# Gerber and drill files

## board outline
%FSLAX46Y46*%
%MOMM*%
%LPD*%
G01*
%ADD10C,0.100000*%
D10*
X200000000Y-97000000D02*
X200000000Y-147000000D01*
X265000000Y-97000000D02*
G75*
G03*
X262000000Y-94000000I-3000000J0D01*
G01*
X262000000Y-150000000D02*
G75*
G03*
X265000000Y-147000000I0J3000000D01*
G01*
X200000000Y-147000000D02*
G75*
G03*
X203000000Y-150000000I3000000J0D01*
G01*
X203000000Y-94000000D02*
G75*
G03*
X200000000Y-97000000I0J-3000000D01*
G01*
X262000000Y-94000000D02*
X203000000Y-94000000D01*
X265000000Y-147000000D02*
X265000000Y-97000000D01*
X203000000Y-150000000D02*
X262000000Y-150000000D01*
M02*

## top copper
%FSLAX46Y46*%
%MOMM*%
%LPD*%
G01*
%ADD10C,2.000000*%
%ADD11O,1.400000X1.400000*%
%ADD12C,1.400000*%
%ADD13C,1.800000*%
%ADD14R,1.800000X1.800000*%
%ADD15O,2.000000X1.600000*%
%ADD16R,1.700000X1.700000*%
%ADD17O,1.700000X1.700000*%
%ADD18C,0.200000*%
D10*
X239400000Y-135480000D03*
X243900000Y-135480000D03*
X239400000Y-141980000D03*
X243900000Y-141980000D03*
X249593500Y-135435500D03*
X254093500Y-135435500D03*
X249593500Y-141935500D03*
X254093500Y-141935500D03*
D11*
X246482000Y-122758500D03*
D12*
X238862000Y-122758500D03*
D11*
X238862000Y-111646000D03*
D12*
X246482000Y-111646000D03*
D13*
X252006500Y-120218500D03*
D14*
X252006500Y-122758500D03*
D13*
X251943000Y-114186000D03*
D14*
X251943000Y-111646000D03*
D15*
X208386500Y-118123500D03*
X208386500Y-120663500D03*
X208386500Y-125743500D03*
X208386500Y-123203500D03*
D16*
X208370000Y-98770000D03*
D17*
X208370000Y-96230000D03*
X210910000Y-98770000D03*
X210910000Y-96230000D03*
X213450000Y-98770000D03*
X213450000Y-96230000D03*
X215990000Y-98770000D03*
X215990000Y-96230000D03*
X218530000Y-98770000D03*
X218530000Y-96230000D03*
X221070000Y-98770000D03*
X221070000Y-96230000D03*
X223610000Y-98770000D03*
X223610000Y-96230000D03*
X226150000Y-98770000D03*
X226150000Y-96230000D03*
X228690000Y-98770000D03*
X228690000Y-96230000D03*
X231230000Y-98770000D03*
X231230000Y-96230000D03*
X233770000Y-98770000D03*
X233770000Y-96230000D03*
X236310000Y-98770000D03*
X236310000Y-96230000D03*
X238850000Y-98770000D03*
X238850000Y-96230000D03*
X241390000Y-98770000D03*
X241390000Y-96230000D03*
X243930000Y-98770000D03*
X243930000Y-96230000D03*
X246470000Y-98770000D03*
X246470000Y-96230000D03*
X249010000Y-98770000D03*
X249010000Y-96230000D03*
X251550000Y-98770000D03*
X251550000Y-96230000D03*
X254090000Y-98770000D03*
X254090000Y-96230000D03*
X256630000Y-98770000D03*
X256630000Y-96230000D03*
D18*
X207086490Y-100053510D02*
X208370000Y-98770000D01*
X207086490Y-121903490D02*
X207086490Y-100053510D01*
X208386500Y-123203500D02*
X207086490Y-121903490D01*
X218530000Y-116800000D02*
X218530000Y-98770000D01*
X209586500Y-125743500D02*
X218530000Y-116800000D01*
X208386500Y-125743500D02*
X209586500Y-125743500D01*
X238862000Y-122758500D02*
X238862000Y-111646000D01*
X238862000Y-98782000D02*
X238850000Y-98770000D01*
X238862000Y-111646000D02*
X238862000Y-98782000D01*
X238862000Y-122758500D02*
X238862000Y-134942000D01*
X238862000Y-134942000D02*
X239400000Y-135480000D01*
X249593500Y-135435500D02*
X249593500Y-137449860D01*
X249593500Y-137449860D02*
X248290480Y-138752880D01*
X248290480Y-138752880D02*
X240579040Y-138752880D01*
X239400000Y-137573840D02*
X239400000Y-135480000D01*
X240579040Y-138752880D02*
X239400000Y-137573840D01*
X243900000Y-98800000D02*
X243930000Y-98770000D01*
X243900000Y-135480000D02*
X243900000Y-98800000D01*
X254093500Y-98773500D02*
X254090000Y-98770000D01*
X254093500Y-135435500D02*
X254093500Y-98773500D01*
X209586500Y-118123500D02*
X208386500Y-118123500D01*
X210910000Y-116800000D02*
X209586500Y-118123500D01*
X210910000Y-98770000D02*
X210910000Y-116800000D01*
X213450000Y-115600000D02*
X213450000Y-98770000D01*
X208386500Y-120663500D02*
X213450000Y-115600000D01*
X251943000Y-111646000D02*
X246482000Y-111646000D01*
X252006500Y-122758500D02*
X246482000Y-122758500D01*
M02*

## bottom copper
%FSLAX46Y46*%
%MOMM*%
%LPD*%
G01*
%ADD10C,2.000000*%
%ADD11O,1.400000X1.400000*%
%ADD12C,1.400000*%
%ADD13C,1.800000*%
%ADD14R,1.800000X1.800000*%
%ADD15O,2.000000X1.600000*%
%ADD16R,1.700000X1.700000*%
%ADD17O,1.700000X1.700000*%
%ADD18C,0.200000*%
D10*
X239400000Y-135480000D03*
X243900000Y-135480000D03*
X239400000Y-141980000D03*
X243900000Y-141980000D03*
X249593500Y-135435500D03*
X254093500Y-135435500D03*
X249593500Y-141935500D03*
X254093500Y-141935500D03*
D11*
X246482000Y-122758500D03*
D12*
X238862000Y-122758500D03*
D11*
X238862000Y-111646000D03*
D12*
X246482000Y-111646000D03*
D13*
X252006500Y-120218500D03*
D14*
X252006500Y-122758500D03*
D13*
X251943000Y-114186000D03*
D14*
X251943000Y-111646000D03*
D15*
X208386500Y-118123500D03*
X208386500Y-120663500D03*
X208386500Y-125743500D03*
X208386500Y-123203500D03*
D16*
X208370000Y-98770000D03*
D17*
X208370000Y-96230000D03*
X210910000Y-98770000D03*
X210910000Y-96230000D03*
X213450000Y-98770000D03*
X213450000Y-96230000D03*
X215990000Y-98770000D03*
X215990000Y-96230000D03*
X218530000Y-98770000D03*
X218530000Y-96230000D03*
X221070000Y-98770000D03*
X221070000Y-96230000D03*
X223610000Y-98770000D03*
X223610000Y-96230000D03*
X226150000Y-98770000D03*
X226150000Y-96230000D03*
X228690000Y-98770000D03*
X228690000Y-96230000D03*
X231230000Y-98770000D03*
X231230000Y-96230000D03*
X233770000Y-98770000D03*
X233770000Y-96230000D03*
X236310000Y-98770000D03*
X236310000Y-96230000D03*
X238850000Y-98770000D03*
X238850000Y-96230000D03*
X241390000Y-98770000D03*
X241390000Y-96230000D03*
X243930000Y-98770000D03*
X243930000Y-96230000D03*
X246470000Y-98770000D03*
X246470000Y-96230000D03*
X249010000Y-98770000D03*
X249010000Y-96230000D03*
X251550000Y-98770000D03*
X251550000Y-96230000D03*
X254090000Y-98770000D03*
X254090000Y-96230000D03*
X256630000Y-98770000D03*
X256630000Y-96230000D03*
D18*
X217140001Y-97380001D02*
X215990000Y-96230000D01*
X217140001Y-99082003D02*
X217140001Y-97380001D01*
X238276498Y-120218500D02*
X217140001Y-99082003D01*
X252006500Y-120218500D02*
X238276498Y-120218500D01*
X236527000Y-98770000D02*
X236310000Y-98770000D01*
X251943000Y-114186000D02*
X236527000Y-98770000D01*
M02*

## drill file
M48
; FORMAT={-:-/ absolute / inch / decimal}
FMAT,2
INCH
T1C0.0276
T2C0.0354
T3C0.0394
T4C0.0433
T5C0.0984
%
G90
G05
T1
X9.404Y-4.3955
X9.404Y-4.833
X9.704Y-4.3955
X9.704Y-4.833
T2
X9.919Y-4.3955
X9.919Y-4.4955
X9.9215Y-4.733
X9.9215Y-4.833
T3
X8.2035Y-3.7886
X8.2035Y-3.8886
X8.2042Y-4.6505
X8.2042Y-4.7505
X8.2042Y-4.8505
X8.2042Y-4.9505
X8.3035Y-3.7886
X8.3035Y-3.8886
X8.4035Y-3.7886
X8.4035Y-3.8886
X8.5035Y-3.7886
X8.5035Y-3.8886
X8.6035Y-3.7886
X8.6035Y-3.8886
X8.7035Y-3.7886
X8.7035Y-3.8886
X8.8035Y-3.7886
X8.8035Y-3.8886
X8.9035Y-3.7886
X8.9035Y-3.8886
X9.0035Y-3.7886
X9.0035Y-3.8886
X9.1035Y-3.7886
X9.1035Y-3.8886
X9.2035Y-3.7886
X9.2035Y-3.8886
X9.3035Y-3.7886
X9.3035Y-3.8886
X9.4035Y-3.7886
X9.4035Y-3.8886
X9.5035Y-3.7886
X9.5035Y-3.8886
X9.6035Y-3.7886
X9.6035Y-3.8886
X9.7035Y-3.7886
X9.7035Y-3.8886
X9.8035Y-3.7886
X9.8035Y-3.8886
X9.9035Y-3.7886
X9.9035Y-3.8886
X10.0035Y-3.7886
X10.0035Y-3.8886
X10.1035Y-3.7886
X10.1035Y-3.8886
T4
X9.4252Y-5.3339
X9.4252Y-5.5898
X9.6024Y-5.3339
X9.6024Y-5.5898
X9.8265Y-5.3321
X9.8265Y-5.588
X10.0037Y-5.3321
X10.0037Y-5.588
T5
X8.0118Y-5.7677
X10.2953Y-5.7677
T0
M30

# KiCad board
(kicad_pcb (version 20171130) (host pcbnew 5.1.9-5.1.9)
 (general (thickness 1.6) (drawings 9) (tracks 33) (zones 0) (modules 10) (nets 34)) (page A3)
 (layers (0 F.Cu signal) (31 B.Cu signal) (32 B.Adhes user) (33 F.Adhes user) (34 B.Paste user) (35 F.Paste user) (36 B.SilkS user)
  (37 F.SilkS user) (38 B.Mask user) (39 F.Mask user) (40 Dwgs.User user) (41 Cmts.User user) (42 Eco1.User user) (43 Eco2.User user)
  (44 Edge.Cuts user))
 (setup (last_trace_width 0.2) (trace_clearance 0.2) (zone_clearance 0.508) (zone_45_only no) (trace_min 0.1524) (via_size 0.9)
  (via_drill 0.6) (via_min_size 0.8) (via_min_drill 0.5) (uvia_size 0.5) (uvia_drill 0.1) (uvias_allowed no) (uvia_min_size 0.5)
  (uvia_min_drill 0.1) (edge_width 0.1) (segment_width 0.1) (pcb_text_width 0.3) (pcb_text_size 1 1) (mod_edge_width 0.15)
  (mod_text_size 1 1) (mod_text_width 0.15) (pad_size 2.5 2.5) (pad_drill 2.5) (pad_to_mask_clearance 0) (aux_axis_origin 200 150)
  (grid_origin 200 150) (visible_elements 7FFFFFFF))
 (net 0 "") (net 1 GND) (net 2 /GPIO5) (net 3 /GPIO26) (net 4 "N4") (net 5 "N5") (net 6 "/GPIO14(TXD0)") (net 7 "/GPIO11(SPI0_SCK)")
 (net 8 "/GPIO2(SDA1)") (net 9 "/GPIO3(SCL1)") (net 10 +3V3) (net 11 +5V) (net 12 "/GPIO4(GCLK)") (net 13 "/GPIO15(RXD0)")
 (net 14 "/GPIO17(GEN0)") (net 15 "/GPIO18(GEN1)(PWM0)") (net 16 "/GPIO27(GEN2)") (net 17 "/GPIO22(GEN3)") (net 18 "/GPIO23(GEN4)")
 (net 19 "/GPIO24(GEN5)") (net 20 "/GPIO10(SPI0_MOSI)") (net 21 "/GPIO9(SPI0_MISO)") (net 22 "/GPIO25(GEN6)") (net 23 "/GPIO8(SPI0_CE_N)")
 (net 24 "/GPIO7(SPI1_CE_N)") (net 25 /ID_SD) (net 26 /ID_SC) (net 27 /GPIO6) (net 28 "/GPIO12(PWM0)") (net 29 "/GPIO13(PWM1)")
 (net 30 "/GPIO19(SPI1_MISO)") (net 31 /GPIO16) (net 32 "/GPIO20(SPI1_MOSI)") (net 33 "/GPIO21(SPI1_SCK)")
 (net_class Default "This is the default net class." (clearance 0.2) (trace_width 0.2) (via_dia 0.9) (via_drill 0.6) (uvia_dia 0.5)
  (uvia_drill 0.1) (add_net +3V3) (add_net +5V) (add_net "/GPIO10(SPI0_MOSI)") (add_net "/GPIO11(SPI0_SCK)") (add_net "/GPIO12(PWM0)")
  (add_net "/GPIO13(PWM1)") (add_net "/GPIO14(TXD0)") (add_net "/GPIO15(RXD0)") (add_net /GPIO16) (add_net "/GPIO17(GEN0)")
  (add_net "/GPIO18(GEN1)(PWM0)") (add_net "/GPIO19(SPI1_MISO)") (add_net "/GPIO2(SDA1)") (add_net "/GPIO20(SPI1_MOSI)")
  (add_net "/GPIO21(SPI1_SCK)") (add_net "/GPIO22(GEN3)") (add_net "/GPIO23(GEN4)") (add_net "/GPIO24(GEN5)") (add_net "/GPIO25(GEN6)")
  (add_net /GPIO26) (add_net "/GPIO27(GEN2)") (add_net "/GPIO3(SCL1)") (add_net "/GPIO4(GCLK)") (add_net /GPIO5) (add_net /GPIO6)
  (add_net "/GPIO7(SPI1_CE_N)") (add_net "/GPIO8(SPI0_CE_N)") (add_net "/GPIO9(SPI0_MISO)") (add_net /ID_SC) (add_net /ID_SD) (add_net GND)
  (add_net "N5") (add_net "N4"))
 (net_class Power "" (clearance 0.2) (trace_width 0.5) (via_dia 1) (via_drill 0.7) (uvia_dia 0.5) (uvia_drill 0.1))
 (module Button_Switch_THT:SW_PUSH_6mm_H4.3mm (layer F.Cu) (at 239.4 141.98 90)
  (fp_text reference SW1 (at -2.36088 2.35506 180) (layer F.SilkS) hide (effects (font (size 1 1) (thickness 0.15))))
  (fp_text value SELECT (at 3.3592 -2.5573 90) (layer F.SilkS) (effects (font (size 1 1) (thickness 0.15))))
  (pad 1 thru_hole circle (at 6.5 0 180) (size 2 2) (drill 1.1) (layers *.Cu *.Mask) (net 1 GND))
  (pad 2 thru_hole circle (at 6.5 4.5 180) (size 2 2) (drill 1.1) (layers *.Cu *.Mask) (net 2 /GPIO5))
  (pad 1 thru_hole circle (at 0 0 180) (size 2 2) (drill 1.1) (layers *.Cu *.Mask) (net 1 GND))
  (pad 2 thru_hole circle (at 0 4.5 180) (size 2 2) (drill 1.1) (layers *.Cu *.Mask) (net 2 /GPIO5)))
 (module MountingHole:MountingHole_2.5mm (layer F.Cu) (at 261.5 146.5)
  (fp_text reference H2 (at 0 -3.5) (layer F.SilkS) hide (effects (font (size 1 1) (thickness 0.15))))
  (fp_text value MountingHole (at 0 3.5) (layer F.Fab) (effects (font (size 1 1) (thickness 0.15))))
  (pad 1 np_thru_hole circle (at 0 0) (size 2.5 2.5) (drill 2.5) (layers *.Cu *.Mask)))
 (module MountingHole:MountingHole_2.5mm (layer F.Cu) (at 203.5 146.5)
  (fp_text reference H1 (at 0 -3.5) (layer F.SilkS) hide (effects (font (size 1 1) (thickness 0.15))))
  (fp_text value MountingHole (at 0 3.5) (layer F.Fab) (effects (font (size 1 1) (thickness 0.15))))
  (pad 1 np_thru_hole circle (at 0 0) (size 2.5 2.5) (drill 2.5) (layers *.Cu *.Mask)))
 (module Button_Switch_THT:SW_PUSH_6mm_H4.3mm (layer F.Cu) (at 249.5935 141.9355 90)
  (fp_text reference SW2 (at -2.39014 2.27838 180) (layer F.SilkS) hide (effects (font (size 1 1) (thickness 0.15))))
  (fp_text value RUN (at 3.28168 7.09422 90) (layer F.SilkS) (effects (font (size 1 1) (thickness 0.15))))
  (pad 1 thru_hole circle (at 6.5 0 180) (size 2 2) (drill 1.1) (layers *.Cu *.Mask) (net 1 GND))
  (pad 2 thru_hole circle (at 6.5 4.5 180) (size 2 2) (drill 1.1) (layers *.Cu *.Mask) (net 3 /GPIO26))
  (pad 1 thru_hole circle (at 0 0 180) (size 2 2) (drill 1.1) (layers *.Cu *.Mask) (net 1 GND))
  (pad 2 thru_hole circle (at 0 4.5 180) (size 2 2) (drill 1.1) (layers *.Cu *.Mask) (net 3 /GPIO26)))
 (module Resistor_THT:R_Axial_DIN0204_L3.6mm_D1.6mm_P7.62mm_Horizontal (layer F.Cu) (at 238.862 122.7585)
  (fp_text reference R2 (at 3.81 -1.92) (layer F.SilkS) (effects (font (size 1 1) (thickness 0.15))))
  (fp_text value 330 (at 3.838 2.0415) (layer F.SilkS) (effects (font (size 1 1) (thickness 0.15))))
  (pad 2 thru_hole oval (at 7.62 0) (size 1.4 1.4) (drill 0.7) (layers *.Cu *.Mask) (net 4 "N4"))
  (pad 1 thru_hole circle (at 0 0) (size 1.4 1.4) (drill 0.7) (layers *.Cu *.Mask) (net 1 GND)))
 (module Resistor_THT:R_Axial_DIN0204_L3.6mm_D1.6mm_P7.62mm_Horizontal (layer F.Cu) (at 246.482 111.646 180)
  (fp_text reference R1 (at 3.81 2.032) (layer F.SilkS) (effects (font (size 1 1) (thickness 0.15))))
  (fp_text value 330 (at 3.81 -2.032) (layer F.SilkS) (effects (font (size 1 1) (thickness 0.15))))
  (pad 2 thru_hole oval (at 7.62 0 180) (size 1.4 1.4) (drill 0.7) (layers *.Cu *.Mask) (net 1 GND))
  (pad 1 thru_hole circle (at 0 0 180) (size 1.4 1.4) (drill 0.7) (layers *.Cu *.Mask) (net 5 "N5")))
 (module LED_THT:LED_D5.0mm (layer F.Cu) (at 252.0065 122.7585 90)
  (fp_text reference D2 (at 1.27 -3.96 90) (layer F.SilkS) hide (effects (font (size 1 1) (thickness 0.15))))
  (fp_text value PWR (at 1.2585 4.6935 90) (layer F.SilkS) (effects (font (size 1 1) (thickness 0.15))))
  (pad 2 thru_hole circle (at 2.54 0 90) (size 1.8 1.8) (drill 0.9) (layers *.Cu *.Mask) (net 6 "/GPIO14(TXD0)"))
  (pad 1 thru_hole rect (at 0 0 90) (size 1.8 1.8) (drill 0.9) (layers *.Cu *.Mask) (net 4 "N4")))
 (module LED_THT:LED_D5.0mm (layer F.Cu) (at 251.943 111.646 270)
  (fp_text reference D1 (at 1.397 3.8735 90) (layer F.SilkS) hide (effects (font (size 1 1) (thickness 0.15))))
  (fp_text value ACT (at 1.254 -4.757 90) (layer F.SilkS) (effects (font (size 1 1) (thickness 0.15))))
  (pad 2 thru_hole circle (at 2.54 0 270) (size 1.8 1.8) (drill 0.9) (layers *.Cu *.Mask) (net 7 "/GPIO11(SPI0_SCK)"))
  (pad 1 thru_hole rect (at 0 0 270) (size 1.8 1.8) (drill 0.9) (layers *.Cu *.Mask) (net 5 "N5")))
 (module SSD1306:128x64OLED (layer F.Cu) (at 218.9865 122.1235 90)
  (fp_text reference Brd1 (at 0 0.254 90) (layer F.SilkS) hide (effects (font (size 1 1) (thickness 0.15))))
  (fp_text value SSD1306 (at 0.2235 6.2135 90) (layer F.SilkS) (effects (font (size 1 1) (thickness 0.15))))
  (pad 4 thru_hole oval (at 4 -10.6 180) (size 2 1.6) (drill 1) (layers *.Cu *.Mask) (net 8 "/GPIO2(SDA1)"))
  (pad 3 thru_hole oval (at 1.46 -10.6 180) (size 2 1.6) (drill 1) (layers *.Cu *.Mask) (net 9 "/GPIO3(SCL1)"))
  (pad 1 thru_hole oval (at -3.62 -10.6 180) (size 2 1.6) (drill 1) (layers *.Cu *.Mask) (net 1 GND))
  (pad 2 thru_hole oval (at -1.08 -10.6 180) (size 2 1.6) (drill 1) (layers *.Cu *.Mask) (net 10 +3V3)))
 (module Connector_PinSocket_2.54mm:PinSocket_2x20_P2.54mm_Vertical (layer B.Cu) (at 208.37 98.77 270)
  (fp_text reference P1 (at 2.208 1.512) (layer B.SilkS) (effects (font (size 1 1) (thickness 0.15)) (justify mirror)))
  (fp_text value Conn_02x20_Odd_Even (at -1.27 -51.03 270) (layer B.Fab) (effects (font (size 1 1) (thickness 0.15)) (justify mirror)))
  (pad 1 thru_hole rect (at 0 0 270) (size 1.7 1.7) (drill 1) (layers *.Cu *.Mask) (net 10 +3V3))
  (pad 2 thru_hole oval (at -2.54 0 270) (size 1.7 1.7) (drill 1) (layers *.Cu *.Mask) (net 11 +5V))
  (pad 3 thru_hole oval (at 0 -2.54 270) (size 1.7 1.7) (drill 1) (layers *.Cu *.Mask) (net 8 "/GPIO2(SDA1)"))
  (pad 4 thru_hole oval (at -2.54 -2.54 270) (size 1.7 1.7) (drill 1) (layers *.Cu *.Mask) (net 11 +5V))
  (pad 5 thru_hole oval (at 0 -5.08 270) (size 1.7 1.7) (drill 1) (layers *.Cu *.Mask) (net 9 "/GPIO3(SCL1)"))
  (pad 6 thru_hole oval (at -2.54 -5.08 270) (size 1.7 1.7) (drill 1) (layers *.Cu *.Mask) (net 1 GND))
  (pad 7 thru_hole oval (at 0 -7.62 270) (size 1.7 1.7) (drill 1) (layers *.Cu *.Mask) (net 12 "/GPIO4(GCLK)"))
  (pad 8 thru_hole oval (at -2.54 -7.62 270) (size 1.7 1.7) (drill 1) (layers *.Cu *.Mask) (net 6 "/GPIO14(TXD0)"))
  (pad 9 thru_hole oval (at 0 -10.16 270) (size 1.7 1.7) (drill 1) (layers *.Cu *.Mask) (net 1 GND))
  (pad 10 thru_hole oval (at -2.54 -10.16 270) (size 1.7 1.7) (drill 1) (layers *.Cu *.Mask) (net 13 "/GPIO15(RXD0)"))
  (pad 11 thru_hole oval (at 0 -12.7 270) (size 1.7 1.7) (drill 1) (layers *.Cu *.Mask) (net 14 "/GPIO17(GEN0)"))
  (pad 12 thru_hole oval (at -2.54 -12.7 270) (size 1.7 1.7) (drill 1) (layers *.Cu *.Mask) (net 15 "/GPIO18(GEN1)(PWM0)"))
  (pad 13 thru_hole oval (at 0 -15.24 270) (size 1.7 1.7) (drill 1) (layers *.Cu *.Mask) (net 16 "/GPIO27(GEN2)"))
  (pad 14 thru_hole oval (at -2.54 -15.24 270) (size 1.7 1.7) (drill 1) (layers *.Cu *.Mask) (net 1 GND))
  (pad 15 thru_hole oval (at 0 -17.78 270) (size 1.7 1.7) (drill 1) (layers *.Cu *.Mask) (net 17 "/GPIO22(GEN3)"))
  (pad 16 thru_hole oval (at -2.54 -17.78 270) (size 1.7 1.7) (drill 1) (layers *.Cu *.Mask) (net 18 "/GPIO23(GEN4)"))
  (pad 17 thru_hole oval (at 0 -20.32 270) (size 1.7 1.7) (drill 1) (layers *.Cu *.Mask) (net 10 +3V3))
  (pad 18 thru_hole oval (at -2.54 -20.32 270) (size 1.7 1.7) (drill 1) (layers *.Cu *.Mask) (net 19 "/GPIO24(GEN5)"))
  (pad 19 thru_hole oval (at 0 -22.86 270) (size 1.7 1.7) (drill 1) (layers *.Cu *.Mask) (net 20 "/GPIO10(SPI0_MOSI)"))
  (pad 20 thru_hole oval (at -2.54 -22.86 270) (size 1.7 1.7) (drill 1) (layers *.Cu *.Mask) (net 1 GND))
  (pad 21 thru_hole oval (at 0 -25.4 270) (size 1.7 1.7) (drill 1) (layers *.Cu *.Mask) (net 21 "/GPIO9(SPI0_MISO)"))
  (pad 22 thru_hole oval (at -2.54 -25.4 270) (size 1.7 1.7) (drill 1) (layers *.Cu *.Mask) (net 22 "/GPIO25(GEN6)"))
  (pad 23 thru_hole oval (at 0 -27.94 270) (size 1.7 1.7) (drill 1) (layers *.Cu *.Mask) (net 7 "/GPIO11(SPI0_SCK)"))
  (pad 24 thru_hole oval (at -2.54 -27.94 270) (size 1.7 1.7) (drill 1) (layers *.Cu *.Mask) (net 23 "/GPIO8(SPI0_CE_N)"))
  (pad 25 thru_hole oval (at 0 -30.48 270) (size 1.7 1.7) (drill 1) (layers *.Cu *.Mask) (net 1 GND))
  (pad 26 thru_hole oval (at -2.54 -30.48 270) (size 1.7 1.7) (drill 1) (layers *.Cu *.Mask) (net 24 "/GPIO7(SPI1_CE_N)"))
  (pad 27 thru_hole oval (at 0 -33.02 270) (size 1.7 1.7) (drill 1) (layers *.Cu *.Mask) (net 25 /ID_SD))
  (pad 28 thru_hole oval (at -2.54 -33.02 270) (size 1.7 1.7) (drill 1) (layers *.Cu *.Mask) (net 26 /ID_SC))
  (pad 29 thru_hole oval (at 0 -35.56 270) (size 1.7 1.7) (drill 1) (layers *.Cu *.Mask) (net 2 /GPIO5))
  (pad 30 thru_hole oval (at -2.54 -35.56 270) (size 1.7 1.7) (drill 1) (layers *.Cu *.Mask) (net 1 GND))
  (pad 31 thru_hole oval (at 0 -38.1 270) (size 1.7 1.7) (drill 1) (layers *.Cu *.Mask) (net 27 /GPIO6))
  (pad 32 thru_hole oval (at -2.54 -38.1 270) (size 1.7 1.7) (drill 1) (layers *.Cu *.Mask) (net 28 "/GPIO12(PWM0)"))
  (pad 33 thru_hole oval (at 0 -40.64 270) (size 1.7 1.7) (drill 1) (layers *.Cu *.Mask) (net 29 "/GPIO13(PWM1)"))
  (pad 34 thru_hole oval (at -2.54 -40.64 270) (size 1.7 1.7) (drill 1) (layers *.Cu *.Mask) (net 1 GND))
  (pad 35 thru_hole oval (at 0 -43.18 270) (size 1.7 1.7) (drill 1) (layers *.Cu *.Mask) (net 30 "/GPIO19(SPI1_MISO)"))
  (pad 36 thru_hole oval (at -2.54 -43.18 270) (size 1.7 1.7) (drill 1) (layers *.Cu *.Mask) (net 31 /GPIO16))
  (pad 37 thru_hole oval (at 0 -45.72 270) (size 1.7 1.7) (drill 1) (layers *.Cu *.Mask) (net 3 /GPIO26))
  (pad 38 thru_hole oval (at -2.54 -45.72 270) (size 1.7 1.7) (drill 1) (layers *.Cu *.Mask) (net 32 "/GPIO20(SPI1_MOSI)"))
  (pad 39 thru_hole oval (at 0 -48.26 270) (size 1.7 1.7) (drill 1) (layers *.Cu *.Mask) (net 1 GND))
  (pad 40 thru_hole oval (at -2.54 -48.26 270) (size 1.7 1.7) (drill 1) (layers *.Cu *.Mask) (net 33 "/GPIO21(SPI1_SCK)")))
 (gr_line (start 200 97) (end 200 147) (layer Edge.Cuts) (width 0.1))
 (gr_arc (start 262 97) (end 262 94) (angle 90) (layer Edge.Cuts) (width 0.1))
 (gr_arc (start 262 147) (end 265 147) (angle 90) (layer Edge.Cuts) (width 0.1))
 (gr_arc (start 203 147) (end 203 150) (angle 90) (layer Edge.Cuts) (width 0.1))
 (gr_arc (start 203 97) (end 200 97) (angle 90) (layer Edge.Cuts) (width 0.1))
 (gr_line (start 262 94) (end 203 94) (layer Edge.Cuts) (width 0.1))
 (gr_line (start 265 147) (end 265 97) (layer Edge.Cuts) (width 0.1))
 (gr_line (start 203 150) (end 262 150) (layer Edge.Cuts) (width 0.1))
 (segment (start 207.08649 100.05351) (end 208.37 98.77) (width 0.2) (layer F.Cu) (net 10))
 (segment (start 207.08649 121.90349) (end 207.08649 100.05351) (width 0.2) (layer F.Cu) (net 10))
 (segment (start 208.3865 123.2035) (end 207.08649 121.90349) (width 0.2) (layer F.Cu) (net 10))
 (segment (start 218.53 116.8) (end 218.53 98.77) (width 0.2) (layer F.Cu) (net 1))
 (segment (start 209.5865 125.7435) (end 218.53 116.8) (width 0.2) (layer F.Cu) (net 1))
 (segment (start 208.3865 125.7435) (end 209.5865 125.7435) (width 0.2) (layer F.Cu) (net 1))
 (segment (start 238.862 122.7585) (end 238.862 111.646) (width 0.2) (layer F.Cu) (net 1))
 (segment (start 238.862 98.782) (end 238.85 98.77) (width 0.2) (layer F.Cu) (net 1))
 (segment (start 238.862 111.646) (end 238.862 98.782) (width 0.2) (layer F.Cu) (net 1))
 (segment (start 238.862 122.7585) (end 238.862 134.942) (width 0.2) (layer F.Cu) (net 1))
 (segment (start 238.862 134.942) (end 239.4 135.48) (width 0.2) (layer F.Cu) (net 1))
 (segment (start 249.5935 135.4355) (end 249.5935 137.44986) (width 0.2) (layer F.Cu) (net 1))
 (segment (start 249.5935 137.44986) (end 248.29048 138.75288) (width 0.2) (layer F.Cu) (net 1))
 (segment (start 248.29048 138.75288) (end 240.57904 138.75288) (width 0.2) (layer F.Cu) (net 1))
 (segment (start 239.4 137.57384) (end 239.4 135.48) (width 0.2) (layer F.Cu) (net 1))
 (segment (start 240.57904 138.75288) (end 239.4 137.57384) (width 0.2) (layer F.Cu) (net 1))
 (segment (start 243.9 98.8) (end 243.93 98.77) (width 0.2) (layer F.Cu) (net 2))
 (segment (start 243.9 135.48) (end 243.9 98.8) (width 0.2) (layer F.Cu) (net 2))
 (segment (start 254.0935 98.7735) (end 254.09 98.77) (width 0.2) (layer F.Cu) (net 3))
 (segment (start 254.0935 135.4355) (end 254.0935 98.7735) (width 0.2) (layer F.Cu) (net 3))
 (segment (start 209.5865 118.1235) (end 208.3865 118.1235) (width 0.2) (layer F.Cu) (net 8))
 (segment (start 210.91 116.8) (end 209.5865 118.1235) (width 0.2) (layer F.Cu) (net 8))
 (segment (start 210.91 98.77) (end 210.91 116.8) (width 0.2) (layer F.Cu) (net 8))
 (segment (start 213.45 115.6) (end 213.45 98.77) (width 0.2) (layer F.Cu) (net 9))
 (segment (start 208.3865 120.6635) (end 213.45 115.6) (width 0.2) (layer F.Cu) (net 9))
 (segment (start 217.140001 97.380001) (end 215.99 96.23) (width 0.2) (layer B.Cu) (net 6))
 (segment (start 217.140001 99.082003) (end 217.140001 97.380001) (width 0.2) (layer B.Cu) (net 6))
 (segment (start 238.276498 120.2185) (end 217.140001 99.082003) (width 0.2) (layer B.Cu) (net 6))
 (segment (start 252.0065 120.2185) (end 238.276498 120.2185) (width 0.2) (layer B.Cu) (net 6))
 (segment (start 236.527 98.77) (end 236.31 98.77) (width 0.2) (layer B.Cu) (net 7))
 (segment (start 251.943 114.186) (end 236.527 98.77) (width 0.2) (layer B.Cu) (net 7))
 (segment (start 251.943 111.646) (end 246.482 111.646) (width 0.2) (layer F.Cu) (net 5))
 (segment (start 252.0065 122.7585) (end 246.482 122.7585) (width 0.2) (layer F.Cu) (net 4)))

